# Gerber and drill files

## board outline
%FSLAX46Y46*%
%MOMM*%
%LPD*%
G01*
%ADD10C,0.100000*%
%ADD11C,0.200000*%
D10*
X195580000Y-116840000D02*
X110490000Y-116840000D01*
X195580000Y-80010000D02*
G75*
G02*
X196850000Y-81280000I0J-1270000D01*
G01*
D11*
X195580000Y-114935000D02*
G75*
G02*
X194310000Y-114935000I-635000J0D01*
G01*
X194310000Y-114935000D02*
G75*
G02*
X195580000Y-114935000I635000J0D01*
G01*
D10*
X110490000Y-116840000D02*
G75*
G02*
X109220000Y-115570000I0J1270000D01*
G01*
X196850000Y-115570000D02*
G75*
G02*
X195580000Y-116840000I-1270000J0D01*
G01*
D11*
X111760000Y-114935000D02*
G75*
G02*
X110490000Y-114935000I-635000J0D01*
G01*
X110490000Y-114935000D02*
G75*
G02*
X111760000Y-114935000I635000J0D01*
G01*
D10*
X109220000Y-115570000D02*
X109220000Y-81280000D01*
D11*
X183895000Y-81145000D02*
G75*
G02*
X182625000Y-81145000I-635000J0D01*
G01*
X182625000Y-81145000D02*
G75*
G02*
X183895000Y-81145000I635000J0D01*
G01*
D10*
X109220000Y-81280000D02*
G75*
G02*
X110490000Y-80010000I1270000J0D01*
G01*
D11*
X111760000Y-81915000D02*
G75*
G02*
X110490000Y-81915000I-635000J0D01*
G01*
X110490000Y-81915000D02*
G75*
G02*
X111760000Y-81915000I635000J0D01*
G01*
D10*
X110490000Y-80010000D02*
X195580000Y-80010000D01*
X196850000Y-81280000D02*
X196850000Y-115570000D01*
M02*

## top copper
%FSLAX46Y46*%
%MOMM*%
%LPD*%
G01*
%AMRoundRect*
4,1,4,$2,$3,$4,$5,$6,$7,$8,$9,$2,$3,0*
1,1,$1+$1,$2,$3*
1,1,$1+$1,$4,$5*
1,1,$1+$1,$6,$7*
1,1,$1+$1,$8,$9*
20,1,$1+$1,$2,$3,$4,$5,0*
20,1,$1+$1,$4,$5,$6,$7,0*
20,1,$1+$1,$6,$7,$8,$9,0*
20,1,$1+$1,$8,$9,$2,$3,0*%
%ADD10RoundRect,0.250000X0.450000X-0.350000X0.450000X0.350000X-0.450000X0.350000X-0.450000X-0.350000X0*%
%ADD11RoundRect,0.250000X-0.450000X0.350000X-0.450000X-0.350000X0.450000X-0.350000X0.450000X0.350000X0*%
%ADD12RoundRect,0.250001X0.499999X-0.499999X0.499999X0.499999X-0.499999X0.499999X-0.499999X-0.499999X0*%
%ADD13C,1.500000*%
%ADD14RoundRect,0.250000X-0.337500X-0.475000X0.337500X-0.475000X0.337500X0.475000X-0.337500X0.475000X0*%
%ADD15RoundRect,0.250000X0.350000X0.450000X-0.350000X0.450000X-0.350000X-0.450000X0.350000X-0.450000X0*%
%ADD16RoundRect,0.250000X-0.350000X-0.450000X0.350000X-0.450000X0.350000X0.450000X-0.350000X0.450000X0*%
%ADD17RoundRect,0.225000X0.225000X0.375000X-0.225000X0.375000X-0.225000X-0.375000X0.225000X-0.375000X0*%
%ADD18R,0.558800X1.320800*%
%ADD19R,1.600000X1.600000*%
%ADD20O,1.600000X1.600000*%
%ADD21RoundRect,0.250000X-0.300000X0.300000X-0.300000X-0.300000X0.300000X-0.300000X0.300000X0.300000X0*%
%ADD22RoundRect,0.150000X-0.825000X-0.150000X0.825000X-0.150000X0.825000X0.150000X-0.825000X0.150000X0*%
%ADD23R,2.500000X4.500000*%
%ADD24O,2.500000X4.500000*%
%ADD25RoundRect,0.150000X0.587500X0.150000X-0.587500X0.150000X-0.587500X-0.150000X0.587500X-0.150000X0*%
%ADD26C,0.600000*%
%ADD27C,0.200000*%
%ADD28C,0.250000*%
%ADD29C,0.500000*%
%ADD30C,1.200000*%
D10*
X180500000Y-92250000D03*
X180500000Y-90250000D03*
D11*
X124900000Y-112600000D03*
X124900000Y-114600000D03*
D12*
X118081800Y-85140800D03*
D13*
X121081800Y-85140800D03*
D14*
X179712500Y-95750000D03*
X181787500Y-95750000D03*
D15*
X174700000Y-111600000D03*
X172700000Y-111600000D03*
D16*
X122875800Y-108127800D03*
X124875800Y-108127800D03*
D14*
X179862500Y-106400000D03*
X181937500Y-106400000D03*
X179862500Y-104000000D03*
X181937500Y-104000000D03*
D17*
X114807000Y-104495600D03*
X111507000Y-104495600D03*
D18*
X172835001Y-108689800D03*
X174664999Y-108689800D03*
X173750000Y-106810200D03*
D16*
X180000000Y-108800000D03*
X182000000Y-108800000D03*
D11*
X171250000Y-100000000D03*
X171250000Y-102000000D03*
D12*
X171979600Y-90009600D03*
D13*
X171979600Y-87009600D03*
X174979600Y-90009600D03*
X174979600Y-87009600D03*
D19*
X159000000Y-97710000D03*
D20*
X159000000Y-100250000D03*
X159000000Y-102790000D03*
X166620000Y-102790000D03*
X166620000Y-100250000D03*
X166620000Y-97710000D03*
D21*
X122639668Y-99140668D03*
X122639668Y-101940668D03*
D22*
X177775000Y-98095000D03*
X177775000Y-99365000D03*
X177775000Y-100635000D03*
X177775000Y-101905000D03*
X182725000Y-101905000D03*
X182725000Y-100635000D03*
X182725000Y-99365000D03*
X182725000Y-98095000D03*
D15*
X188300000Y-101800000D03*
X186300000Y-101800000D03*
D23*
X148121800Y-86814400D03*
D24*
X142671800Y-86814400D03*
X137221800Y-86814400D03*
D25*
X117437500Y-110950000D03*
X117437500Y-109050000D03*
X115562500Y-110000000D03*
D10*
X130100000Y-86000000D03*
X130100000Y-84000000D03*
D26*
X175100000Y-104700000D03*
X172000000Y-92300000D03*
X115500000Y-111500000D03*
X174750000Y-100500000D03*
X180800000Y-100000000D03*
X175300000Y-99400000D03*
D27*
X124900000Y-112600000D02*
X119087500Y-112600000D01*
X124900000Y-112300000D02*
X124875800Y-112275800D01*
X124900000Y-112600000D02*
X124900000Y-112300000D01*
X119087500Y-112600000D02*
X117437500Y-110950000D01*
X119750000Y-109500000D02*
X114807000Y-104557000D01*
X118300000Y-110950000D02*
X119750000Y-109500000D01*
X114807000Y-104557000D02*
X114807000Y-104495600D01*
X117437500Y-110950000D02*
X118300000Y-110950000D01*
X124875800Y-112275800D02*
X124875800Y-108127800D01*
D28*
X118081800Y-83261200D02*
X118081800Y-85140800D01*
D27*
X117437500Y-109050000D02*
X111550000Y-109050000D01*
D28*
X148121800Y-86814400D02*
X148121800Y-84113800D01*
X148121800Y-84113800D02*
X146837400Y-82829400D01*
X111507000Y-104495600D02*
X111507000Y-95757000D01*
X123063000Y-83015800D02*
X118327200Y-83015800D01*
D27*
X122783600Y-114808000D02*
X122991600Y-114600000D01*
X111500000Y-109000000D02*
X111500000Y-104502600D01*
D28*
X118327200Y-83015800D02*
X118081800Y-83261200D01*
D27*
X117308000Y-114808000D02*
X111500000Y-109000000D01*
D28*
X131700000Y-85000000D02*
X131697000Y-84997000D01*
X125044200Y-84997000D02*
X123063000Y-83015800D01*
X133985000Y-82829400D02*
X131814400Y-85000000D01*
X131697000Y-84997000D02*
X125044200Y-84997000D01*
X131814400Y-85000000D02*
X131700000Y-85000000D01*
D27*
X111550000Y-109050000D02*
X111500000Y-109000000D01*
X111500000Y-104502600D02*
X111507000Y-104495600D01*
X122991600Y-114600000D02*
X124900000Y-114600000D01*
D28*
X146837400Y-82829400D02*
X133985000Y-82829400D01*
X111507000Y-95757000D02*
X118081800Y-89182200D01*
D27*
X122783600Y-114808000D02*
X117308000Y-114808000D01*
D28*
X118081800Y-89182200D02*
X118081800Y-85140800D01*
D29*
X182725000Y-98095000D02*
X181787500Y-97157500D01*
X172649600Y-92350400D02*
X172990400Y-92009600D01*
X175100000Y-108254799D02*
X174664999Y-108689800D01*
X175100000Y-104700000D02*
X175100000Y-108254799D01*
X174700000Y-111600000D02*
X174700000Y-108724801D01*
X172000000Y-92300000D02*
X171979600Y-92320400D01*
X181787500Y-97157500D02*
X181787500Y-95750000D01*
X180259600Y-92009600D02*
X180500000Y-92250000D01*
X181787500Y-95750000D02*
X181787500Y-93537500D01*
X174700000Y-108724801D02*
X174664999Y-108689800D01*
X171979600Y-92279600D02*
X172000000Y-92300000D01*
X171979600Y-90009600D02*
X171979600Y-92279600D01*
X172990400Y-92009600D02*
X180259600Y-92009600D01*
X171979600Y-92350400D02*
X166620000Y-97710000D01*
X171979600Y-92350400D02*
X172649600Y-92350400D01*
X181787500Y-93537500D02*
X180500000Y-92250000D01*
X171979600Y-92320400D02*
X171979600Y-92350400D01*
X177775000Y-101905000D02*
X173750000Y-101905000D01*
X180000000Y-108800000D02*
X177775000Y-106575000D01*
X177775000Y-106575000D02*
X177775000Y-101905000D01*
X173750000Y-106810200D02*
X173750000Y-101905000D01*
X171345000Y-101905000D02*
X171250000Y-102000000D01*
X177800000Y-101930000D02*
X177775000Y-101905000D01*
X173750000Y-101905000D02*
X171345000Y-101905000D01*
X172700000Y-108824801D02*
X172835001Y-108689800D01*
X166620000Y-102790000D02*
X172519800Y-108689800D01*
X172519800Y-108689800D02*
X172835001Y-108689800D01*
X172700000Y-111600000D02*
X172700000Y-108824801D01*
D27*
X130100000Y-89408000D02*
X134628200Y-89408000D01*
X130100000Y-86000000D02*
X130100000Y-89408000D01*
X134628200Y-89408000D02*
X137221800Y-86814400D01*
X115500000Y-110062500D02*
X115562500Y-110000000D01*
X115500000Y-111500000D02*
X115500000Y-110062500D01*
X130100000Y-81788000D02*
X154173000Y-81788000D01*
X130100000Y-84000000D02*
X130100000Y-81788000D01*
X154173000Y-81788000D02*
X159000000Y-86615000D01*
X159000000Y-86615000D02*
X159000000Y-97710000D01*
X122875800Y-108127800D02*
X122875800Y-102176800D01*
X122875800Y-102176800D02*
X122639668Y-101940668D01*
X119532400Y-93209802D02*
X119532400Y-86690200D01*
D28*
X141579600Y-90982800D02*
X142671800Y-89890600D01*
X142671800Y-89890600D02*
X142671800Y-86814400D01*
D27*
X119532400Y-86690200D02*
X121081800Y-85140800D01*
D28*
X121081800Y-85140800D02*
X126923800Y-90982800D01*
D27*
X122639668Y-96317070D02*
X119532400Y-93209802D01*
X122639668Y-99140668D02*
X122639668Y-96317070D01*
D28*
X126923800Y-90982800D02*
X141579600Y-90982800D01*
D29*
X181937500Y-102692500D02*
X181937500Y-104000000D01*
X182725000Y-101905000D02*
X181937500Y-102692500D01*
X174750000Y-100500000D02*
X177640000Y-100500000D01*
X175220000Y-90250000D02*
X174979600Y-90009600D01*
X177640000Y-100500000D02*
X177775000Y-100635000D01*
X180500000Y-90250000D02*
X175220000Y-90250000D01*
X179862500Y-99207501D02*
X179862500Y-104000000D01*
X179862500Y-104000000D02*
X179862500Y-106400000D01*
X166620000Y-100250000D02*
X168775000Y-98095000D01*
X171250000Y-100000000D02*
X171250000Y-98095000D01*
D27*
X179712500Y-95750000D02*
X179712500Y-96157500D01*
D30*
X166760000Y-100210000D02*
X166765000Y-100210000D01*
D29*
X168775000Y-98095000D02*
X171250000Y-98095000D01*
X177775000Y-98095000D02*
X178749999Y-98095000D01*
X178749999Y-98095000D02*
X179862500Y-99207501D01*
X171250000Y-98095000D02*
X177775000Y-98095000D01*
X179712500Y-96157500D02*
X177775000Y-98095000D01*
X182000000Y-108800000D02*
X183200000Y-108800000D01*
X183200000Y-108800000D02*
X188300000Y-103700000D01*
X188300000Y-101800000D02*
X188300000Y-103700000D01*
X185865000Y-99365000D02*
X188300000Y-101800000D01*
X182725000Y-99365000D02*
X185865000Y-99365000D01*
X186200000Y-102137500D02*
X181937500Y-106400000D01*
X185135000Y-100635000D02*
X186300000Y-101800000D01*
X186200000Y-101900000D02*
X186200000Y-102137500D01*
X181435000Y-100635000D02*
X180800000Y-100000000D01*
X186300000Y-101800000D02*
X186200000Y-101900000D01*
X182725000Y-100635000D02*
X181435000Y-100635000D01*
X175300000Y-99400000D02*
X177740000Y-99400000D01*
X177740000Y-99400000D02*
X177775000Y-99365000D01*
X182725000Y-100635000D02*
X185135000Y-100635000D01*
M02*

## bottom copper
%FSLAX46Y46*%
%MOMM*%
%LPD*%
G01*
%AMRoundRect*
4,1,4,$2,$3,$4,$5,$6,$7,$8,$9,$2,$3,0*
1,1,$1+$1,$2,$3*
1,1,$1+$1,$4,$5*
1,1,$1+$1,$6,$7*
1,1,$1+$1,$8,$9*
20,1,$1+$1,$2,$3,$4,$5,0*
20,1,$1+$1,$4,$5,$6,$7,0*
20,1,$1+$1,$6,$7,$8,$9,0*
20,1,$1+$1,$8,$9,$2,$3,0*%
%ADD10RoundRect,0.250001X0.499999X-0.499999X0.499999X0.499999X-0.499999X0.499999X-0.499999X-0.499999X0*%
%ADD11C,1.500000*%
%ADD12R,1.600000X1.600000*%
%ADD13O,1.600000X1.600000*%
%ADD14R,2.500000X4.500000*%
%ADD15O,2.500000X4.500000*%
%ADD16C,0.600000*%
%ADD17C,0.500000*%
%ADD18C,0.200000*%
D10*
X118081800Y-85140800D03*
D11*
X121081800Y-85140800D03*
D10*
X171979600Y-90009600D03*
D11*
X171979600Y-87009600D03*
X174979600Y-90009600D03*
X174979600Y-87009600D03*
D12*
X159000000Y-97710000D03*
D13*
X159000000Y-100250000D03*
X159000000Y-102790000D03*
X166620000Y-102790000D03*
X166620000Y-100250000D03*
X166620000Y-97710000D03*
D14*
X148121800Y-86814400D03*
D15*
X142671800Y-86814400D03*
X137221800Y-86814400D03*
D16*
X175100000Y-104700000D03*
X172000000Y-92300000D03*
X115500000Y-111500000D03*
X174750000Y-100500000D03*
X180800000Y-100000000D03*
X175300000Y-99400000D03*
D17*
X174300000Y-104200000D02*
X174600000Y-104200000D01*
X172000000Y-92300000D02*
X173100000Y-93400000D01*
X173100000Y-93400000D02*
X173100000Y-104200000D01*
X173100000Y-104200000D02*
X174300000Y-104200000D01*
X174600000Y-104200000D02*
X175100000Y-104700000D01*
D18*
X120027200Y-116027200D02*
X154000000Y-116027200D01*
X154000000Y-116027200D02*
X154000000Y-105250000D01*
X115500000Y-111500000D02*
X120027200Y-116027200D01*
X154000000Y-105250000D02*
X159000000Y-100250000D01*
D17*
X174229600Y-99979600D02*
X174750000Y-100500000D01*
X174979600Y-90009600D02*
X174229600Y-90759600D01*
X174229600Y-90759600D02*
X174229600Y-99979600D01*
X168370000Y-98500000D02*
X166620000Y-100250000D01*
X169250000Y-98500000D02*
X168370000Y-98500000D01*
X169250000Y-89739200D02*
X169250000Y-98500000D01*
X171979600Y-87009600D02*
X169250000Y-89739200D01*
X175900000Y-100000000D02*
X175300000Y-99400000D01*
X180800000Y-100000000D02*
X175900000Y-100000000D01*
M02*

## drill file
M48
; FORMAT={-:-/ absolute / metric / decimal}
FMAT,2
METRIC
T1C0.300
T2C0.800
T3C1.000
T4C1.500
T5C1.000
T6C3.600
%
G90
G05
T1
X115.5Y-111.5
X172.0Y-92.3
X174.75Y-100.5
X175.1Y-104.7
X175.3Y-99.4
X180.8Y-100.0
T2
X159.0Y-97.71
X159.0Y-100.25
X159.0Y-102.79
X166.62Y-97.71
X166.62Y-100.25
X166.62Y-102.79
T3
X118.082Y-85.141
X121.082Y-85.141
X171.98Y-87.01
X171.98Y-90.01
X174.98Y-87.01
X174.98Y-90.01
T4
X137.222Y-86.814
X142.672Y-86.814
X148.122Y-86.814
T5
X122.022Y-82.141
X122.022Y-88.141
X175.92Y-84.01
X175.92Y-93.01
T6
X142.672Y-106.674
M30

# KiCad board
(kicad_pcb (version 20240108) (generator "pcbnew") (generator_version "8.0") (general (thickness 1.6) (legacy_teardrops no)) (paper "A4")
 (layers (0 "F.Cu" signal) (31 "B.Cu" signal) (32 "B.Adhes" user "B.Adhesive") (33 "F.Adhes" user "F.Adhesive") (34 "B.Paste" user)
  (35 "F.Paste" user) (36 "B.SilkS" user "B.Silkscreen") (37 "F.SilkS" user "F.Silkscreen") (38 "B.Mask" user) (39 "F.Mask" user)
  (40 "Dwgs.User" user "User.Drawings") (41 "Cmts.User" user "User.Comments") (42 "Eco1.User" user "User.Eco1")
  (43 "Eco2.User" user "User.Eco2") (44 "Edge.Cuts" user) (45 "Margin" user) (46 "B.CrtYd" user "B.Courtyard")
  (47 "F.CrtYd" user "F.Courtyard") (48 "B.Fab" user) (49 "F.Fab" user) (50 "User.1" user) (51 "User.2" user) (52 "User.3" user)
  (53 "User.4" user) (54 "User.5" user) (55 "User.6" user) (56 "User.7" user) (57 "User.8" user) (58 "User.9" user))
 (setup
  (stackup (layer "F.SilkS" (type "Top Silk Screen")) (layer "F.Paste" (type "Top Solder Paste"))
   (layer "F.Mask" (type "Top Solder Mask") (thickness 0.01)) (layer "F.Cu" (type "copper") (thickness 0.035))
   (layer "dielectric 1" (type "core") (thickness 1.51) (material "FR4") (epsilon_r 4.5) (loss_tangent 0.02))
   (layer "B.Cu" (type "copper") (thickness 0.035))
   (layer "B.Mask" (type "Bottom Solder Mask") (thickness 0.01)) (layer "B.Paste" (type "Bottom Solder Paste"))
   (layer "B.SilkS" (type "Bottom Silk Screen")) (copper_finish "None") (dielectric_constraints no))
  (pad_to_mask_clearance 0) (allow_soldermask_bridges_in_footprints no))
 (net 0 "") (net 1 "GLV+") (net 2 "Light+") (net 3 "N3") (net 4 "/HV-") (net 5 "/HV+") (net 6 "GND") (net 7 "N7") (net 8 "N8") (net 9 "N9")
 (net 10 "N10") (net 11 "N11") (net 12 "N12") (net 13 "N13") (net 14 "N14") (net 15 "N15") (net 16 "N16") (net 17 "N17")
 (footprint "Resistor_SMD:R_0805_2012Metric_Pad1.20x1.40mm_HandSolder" (layer "F.Cu") (at 180.5 91.25 90)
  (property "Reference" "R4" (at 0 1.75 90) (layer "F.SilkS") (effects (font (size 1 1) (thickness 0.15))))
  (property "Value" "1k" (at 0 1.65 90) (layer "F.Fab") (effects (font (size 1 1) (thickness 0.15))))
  (pad "1" smd roundrect (at -1 0 90) (size 1.2 1.4) (layers "F.Cu" "F.Paste" "F.Mask") (roundrect_rratio 0.208333) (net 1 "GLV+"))
  (pad "2" smd roundrect (at 1 0 90) (size 1.2 1.4) (layers "F.Cu" "F.Paste" "F.Mask") (roundrect_rratio 0.208333) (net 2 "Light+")))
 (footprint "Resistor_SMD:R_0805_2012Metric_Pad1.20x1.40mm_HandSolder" (layer "F.Cu") (at 124.9 113.6 -90)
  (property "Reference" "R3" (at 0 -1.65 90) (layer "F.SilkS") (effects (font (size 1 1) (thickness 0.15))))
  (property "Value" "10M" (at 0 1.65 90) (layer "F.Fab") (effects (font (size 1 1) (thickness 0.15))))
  (pad "1" smd roundrect (at -1 0 270) (size 1.2 1.4) (layers "F.Cu" "F.Paste" "F.Mask") (roundrect_rratio 0.208333) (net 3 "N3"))
  (pad "2" smd roundrect (at 1 0 270) (size 1.2 1.4) (layers "F.Cu" "F.Paste" "F.Mask") (roundrect_rratio 0.208333) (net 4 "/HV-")))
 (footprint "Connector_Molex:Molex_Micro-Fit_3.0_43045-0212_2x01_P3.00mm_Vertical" (layer "F.Cu") (at 118.0818 85.1408 90)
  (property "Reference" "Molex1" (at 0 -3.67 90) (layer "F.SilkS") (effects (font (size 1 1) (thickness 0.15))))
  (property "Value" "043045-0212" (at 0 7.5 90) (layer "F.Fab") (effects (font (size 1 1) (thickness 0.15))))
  (pad "" np_thru_hole circle (at -3 3.94 90) (size 1 1) (drill 1) (layers "*.Cu" "*.Mask"))
  (pad "" np_thru_hole circle (at 3 3.94 90) (size 1 1) (drill 1) (layers "*.Cu" "*.Mask"))
  (pad "1" thru_hole roundrect (at 0 0 90) (size 1.5 1.5) (drill 1) (layers "*.Cu" "*.Mask") (remove_unused_layers no)
   (roundrect_rratio 0.166667) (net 4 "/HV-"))
  (pad "2" thru_hole circle (at 0 3 90) (size 1.5 1.5) (drill 1) (layers "*.Cu" "*.Mask") (remove_unused_layers no) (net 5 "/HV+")))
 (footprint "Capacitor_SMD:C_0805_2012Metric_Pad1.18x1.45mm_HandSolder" (layer "F.Cu") (at 180.75 95.75)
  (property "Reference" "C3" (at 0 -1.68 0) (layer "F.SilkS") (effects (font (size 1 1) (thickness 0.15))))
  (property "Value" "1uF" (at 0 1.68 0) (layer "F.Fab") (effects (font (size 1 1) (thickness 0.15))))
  (pad "1" smd roundrect (at -1.0375 0) (size 1.175 1.45) (layers "F.Cu" "F.Paste" "F.Mask") (roundrect_rratio 0.212766) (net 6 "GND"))
  (pad "2" smd roundrect (at 1.0375 0) (size 1.175 1.45) (layers "F.Cu" "F.Paste" "F.Mask") (roundrect_rratio 0.212766) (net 1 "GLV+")))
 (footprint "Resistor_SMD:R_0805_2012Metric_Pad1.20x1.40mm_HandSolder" (layer "F.Cu") (at 173.7 111.6 180)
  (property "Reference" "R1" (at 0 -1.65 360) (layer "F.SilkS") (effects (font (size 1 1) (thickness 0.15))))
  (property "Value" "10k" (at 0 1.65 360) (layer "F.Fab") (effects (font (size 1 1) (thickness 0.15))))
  (pad "1" smd roundrect (at -1 0 180) (size 1.2 1.4) (layers "F.Cu" "F.Paste" "F.Mask") (roundrect_rratio 0.208333) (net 1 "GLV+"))
  (pad "2" smd roundrect (at 1 0 180) (size 1.2 1.4) (layers "F.Cu" "F.Paste" "F.Mask") (roundrect_rratio 0.208333) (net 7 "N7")))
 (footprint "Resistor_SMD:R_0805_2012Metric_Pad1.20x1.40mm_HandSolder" (layer "F.Cu") (at 123.8758 108.1278)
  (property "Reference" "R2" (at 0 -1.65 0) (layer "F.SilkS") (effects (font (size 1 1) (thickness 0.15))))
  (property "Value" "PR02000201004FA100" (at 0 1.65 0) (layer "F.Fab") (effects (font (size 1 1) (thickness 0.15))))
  (pad "1" smd roundrect (at -1 0) (size 1.2 1.4) (layers "F.Cu" "F.Paste" "F.Mask") (roundrect_rratio 0.208333) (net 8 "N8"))
  (pad "2" smd roundrect (at 1 0) (size 1.2 1.4) (layers "F.Cu" "F.Paste" "F.Mask") (roundrect_rratio 0.208333) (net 3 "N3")))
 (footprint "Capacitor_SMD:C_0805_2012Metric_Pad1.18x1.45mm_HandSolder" (layer "F.Cu") (at 180.9 106.4)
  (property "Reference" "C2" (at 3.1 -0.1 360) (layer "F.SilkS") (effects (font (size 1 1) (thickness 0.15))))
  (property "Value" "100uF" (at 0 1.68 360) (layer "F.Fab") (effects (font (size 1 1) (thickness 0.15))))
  (pad "1" smd roundrect (at -1.0375 0) (size 1.175 1.45) (layers "F.Cu" "F.Paste" "F.Mask") (roundrect_rratio 0.212766) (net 6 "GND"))
  (pad "2" smd roundrect (at 1.0375 0) (size 1.175 1.45) (layers "F.Cu" "F.Paste" "F.Mask") (roundrect_rratio 0.212766) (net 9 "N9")))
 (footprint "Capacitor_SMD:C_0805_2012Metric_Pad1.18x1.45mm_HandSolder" (layer "F.Cu") (at 180.9 104)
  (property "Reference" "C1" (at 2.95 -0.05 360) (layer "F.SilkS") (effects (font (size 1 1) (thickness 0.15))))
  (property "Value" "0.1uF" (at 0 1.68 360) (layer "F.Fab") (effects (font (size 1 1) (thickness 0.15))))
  (pad "1" smd roundrect (at -1.0375 0) (size 1.175 1.45) (layers "F.Cu" "F.Paste" "F.Mask") (roundrect_rratio 0.212766) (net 6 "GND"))
  (pad "2" smd roundrect (at 1.0375 0) (size 1.175 1.45) (layers "F.Cu" "F.Paste" "F.Mask") (roundrect_rratio 0.212766) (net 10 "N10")))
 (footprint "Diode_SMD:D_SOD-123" (layer "F.Cu") (at 113.157 104.4956 180)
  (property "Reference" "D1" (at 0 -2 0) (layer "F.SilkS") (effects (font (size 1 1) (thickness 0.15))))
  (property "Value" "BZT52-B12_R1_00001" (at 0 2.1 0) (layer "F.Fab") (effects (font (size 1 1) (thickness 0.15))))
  (pad "1" smd roundrect (at -1.65 0 180) (size 0.9 1.2) (layers "F.Cu" "F.Paste" "F.Mask") (roundrect_rratio 0.25) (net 3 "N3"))
  (pad "2" smd roundrect (at 1.65 0 180) (size 0.9 1.2) (layers "F.Cu" "F.Paste" "F.Mask") (roundrect_rratio 0.25) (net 4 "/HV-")))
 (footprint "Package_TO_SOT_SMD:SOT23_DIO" (layer "F.Cu") (at 173.75 107.75)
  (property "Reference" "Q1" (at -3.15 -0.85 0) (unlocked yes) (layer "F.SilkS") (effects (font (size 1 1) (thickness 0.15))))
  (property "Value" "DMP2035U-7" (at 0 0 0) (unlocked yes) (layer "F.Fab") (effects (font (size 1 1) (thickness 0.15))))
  (pad "1" smd rect (at -0.914999 0.9398) (size 0.5588 1.3208) (layers "F.Cu" "F.Paste" "F.Mask") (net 7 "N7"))
  (pad "2" smd rect (at 0.914999 0.9398) (size 0.5588 1.3208) (layers "F.Cu" "F.Paste" "F.Mask") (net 1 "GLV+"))
  (pad "3" smd rect (at 0 -0.9398) (size 0.5588 1.3208) (layers "F.Cu" "F.Paste" "F.Mask") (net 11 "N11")))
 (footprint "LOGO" (layer "F.Cu") (at 156.25 108.5)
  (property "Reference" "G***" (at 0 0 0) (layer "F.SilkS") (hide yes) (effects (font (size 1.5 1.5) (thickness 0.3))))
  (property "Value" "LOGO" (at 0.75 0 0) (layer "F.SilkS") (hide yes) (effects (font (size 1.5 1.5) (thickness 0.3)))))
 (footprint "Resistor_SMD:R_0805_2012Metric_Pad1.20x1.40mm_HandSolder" (layer "F.Cu") (at 181 108.8)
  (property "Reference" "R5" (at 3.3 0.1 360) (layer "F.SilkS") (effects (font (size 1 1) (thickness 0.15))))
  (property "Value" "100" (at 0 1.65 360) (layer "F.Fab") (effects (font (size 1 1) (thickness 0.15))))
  (pad "1" smd roundrect (at -1 0) (size 1.2 1.4) (layers "F.Cu" "F.Paste" "F.Mask") (roundrect_rratio 0.208333) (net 11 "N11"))
  (pad "2" smd roundrect (at 1 0) (size 1.2 1.4) (layers "F.Cu" "F.Paste" "F.Mask") (roundrect_rratio 0.208333) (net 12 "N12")))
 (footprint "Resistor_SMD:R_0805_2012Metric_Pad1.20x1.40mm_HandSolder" (layer "F.Cu") (at 171.25 101 -90)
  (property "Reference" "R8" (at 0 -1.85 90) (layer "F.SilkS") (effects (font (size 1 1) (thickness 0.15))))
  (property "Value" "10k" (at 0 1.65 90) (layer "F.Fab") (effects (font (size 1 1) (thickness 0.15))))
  (pad "1" smd roundrect (at -1 0 270) (size 1.2 1.4) (layers "F.Cu" "F.Paste" "F.Mask") (roundrect_rratio 0.208333) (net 6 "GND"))
  (pad "2" smd roundrect (at 1 0 270) (size 1.2 1.4) (layers "F.Cu" "F.Paste" "F.Mask") (roundrect_rratio 0.208333) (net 11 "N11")))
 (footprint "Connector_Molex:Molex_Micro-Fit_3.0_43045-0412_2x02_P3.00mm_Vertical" (layer "F.Cu") (at 171.9796 90.0096 90)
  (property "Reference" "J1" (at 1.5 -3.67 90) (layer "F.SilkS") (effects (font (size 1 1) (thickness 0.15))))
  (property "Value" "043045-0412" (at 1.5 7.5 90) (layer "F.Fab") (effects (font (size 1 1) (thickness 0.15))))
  (pad "" np_thru_hole circle (at -3 3.94 90) (size 1 1) (drill 1) (layers "*.Cu" "*.Mask"))
  (pad "" np_thru_hole circle (at 6 3.94 90) (size 1 1) (drill 1) (layers "*.Cu" "*.Mask"))
  (pad "1" thru_hole roundrect (at 0 0 90) (size 1.5 1.5) (drill 1) (layers "*.Cu" "*.Mask") (remove_unused_layers no)
   (roundrect_rratio 0.166667) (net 1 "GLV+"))
  (pad "2" thru_hole circle (at 3 0 90) (size 1.5 1.5) (drill 1) (layers "*.Cu" "*.Mask") (remove_unused_layers no) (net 6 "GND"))
  (pad "3" thru_hole circle (at 0 3 90) (size 1.5 1.5) (drill 1) (layers "*.Cu" "*.Mask") (remove_unused_layers no) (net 2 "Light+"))
  (pad "4" thru_hole circle (at 3 3 90) (size 1.5 1.5) (drill 1) (layers "*.Cu" "*.Mask") (remove_unused_layers no) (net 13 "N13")))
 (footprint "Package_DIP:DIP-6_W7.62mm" (layer "F.Cu") (at 159 97.71)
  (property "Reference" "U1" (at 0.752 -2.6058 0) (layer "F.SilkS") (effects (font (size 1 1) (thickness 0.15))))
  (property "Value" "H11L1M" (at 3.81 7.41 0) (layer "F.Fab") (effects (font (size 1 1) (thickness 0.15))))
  (pad "1" thru_hole rect (at 0 0) (size 1.6 1.6) (drill 0.8) (layers "*.Cu" "*.Mask") (remove_unused_layers no) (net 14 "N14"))
  (pad "2" thru_hole oval (at 0 2.54) (size 1.6 1.6) (drill 0.8) (layers "*.Cu" "*.Mask") (remove_unused_layers no) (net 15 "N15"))
  (pad "3" thru_hole oval (at 0 5.08) (size 1.6 1.6) (drill 0.8) (layers "*.Cu" "*.Mask") (remove_unused_layers no) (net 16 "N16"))
  (pad "4" thru_hole oval (at 7.62 5.08) (size 1.6 1.6) (drill 0.8) (layers "*.Cu" "*.Mask") (remove_unused_layers no) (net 7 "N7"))
  (pad "5" thru_hole oval (at 7.62 2.54) (size 1.6 1.6) (drill 0.8) (layers "*.Cu" "*.Mask") (remove_unused_layers no) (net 6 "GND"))
  (pad "6" thru_hole oval (at 7.62 0) (size 1.6 1.6) (drill 0.8) (layers "*.Cu" "*.Mask") (remove_unused_layers no) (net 1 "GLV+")))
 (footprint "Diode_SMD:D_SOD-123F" (layer "F.Cu") (at 122.639668 100.540668 -90)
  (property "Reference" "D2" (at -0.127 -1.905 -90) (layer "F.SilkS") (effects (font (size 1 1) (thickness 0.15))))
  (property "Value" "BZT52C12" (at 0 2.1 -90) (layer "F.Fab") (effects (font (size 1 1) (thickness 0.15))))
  (pad "1" smd roundrect (at -1.4 0 270) (size 1.1 1.1) (layers "F.Cu" "F.Paste" "F.Mask") (roundrect_rratio 0.2272727273) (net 5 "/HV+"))
  (pad "2" smd roundrect (at 1.4 0 270) (size 1.1 1.1) (layers "F.Cu" "F.Paste" "F.Mask") (roundrect_rratio 0.2272727273) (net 8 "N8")))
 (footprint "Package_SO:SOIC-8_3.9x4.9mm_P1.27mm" (layer "F.Cu") (at 180.25 100)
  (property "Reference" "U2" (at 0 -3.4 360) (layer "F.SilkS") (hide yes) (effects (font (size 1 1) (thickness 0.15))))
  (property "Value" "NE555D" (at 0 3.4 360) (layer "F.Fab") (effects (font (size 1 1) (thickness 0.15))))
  (pad "1" smd roundrect (at -2.475 -1.905) (size 1.95 0.6) (layers "F.Cu" "F.Paste" "F.Mask") (roundrect_rratio 0.25) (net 6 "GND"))
  (pad "2" smd roundrect (at -2.475 -0.635) (size 1.95 0.6) (layers "F.Cu" "F.Paste" "F.Mask") (roundrect_rratio 0.25) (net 9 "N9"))
  (pad "3" smd roundrect (at -2.475 0.635) (size 1.95 0.6) (layers "F.Cu" "F.Paste" "F.Mask") (roundrect_rratio 0.25) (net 2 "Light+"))
  (pad "4" smd roundrect (at -2.475 1.905) (size 1.95 0.6) (layers "F.Cu" "F.Paste" "F.Mask") (roundrect_rratio 0.25) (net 11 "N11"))
  (pad "5" smd roundrect (at 2.475 1.905) (size 1.95 0.6) (layers "F.Cu" "F.Paste" "F.Mask") (roundrect_rratio 0.25) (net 10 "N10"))
  (pad "6" smd roundrect (at 2.475 0.635) (size 1.95 0.6) (layers "F.Cu" "F.Paste" "F.Mask") (roundrect_rratio 0.25) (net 9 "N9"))
  (pad "7" smd roundrect (at 2.475 -0.635) (size 1.95 0.6) (layers "F.Cu" "F.Paste" "F.Mask") (roundrect_rratio 0.25) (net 12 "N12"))
  (pad "8" smd roundrect (at 2.475 -1.905) (size 1.95 0.6) (layers "F.Cu" "F.Paste" "F.Mask") (roundrect_rratio 0.25) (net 1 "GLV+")))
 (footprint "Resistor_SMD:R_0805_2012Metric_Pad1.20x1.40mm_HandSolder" (layer "F.Cu") (at 187.3 101.8 180)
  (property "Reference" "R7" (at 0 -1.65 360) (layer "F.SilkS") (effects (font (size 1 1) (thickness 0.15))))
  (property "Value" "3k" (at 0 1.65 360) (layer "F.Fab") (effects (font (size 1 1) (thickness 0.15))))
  (pad "1" smd roundrect (at -1 0 180) (size 1.2 1.4) (layers "F.Cu" "F.Paste" "F.Mask") (roundrect_rratio 0.208333) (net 12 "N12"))
  (pad "2" smd roundrect (at 1 0 180) (size 1.2 1.4) (layers "F.Cu" "F.Paste" "F.Mask") (roundrect_rratio 0.208333) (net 9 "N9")))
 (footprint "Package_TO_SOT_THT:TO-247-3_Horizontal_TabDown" (layer "F.Cu") (at 148.1218 86.8144 180)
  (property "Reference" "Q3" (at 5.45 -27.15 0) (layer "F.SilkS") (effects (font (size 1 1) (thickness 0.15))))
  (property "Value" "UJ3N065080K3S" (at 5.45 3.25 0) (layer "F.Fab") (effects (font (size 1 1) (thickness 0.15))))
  (pad "" np_thru_hole oval (at 5.45 -19.86 180) (size 3.6 3.6) (drill 3.6) (layers "*.Cu" "*.Mask"))
  (pad "1" thru_hole rect (at 0 0 180) (size 2.5 4.5) (drill 1.5) (layers "*.Cu" "*.Mask") (remove_unused_layers no) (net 4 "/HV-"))
  (pad "2" thru_hole oval (at 5.45 0 180) (size 2.5 4.5) (drill 1.5) (layers "*.Cu" "*.Mask") (remove_unused_layers no) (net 5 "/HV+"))
  (pad "3" thru_hole oval (at 10.9 0 180) (size 2.5 4.5) (drill 1.5) (layers "*.Cu" "*.Mask") (remove_unused_layers no) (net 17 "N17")))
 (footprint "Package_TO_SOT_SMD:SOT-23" (layer "F.Cu") (at 116.5 110 180)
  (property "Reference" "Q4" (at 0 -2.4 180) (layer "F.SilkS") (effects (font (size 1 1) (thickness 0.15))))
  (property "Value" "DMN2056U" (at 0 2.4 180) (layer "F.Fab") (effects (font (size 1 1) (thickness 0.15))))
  (pad "1" smd roundrect (at -0.9375 -0.95 180) (size 1.475 0.6) (layers "F.Cu" "F.Paste" "F.Mask") (roundrect_rratio 0.25) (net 3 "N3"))
  (pad "2" smd roundrect (at -0.9375 0.95 180) (size 1.475 0.6) (layers "F.Cu" "F.Paste" "F.Mask") (roundrect_rratio 0.25) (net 4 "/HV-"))
  (pad "3" smd roundrect (at 0.9375 0 180) (size 1.475 0.6) (layers "F.Cu" "F.Paste" "F.Mask") (roundrect_rratio 0.25) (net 15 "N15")))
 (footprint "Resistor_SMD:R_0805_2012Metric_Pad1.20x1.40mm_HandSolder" (layer "F.Cu") (at 130.1 85 90)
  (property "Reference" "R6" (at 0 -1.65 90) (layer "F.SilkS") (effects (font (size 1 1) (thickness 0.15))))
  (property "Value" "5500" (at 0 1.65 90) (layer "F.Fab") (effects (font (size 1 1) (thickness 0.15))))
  (pad "1" smd roundrect (at -1 0 90) (size 1.2 1.4) (layers "F.Cu" "F.Paste" "F.Mask") (roundrect_rratio 0.208333) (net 17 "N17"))
  (pad "2" smd roundrect (at 1 0 90) (size 1.2 1.4) (layers "F.Cu" "F.Paste" "F.Mask") (roundrect_rratio 0.208333) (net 14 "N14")))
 (gr_line (start 195.58 116.84) (end 110.49 116.84) (stroke (width 0.1) (type default)) (layer "Edge.Cuts"))
 (gr_arc (start 195.58 80.01) (mid 196.478026 80.381974) (end 196.85 81.28) (stroke (width 0.1) (type default)) (layer "Edge.Cuts"))
 (gr_circle (center 194.945 114.935) (end 195.58 114.935) (stroke (width 0.2) (type default)) (fill none) (layer "Edge.Cuts"))
 (gr_arc (start 110.49 116.84) (mid 109.591974 116.468026) (end 109.22 115.57) (stroke (width 0.1) (type default)) (layer "Edge.Cuts"))
 (gr_arc (start 196.85 115.57) (mid 196.478026 116.468026) (end 195.58 116.84) (stroke (width 0.1) (type default)) (layer "Edge.Cuts"))
 (gr_circle (center 111.125 114.935) (end 111.76 114.935) (stroke (width 0.2) (type default)) (fill none) (layer "Edge.Cuts"))
 (gr_line (start 109.22 115.57) (end 109.22 81.28) (stroke (width 0.1) (type default)) (layer "Edge.Cuts"))
 (gr_circle (center 183.26 81.145) (end 183.895 81.145) (stroke (width 0.2) (type default)) (fill none) (layer "Edge.Cuts"))
 (gr_arc (start 109.22 81.28) (mid 109.591974 80.381974) (end 110.49 80.01) (stroke (width 0.1) (type default)) (layer "Edge.Cuts"))
 (gr_circle (center 111.125 81.915) (end 111.76 81.915) (stroke (width 0.2) (type default)) (fill none) (layer "Edge.Cuts"))
 (gr_line (start 110.49 80.01) (end 195.58 80.01) (stroke (width 0.1) (type default)) (layer "Edge.Cuts"))
 (gr_line (start 196.85 81.28) (end 196.85 115.57) (stroke (width 0.1) (type default)) (layer "Edge.Cuts"))
 (segment (start 124.9 112.6) (end 119.0875 112.6) (width 0.2) (layer "F.Cu") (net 3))
 (segment (start 124.9 112.3) (end 124.8758 112.2758) (width 0.2) (layer "F.Cu") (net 3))
 (segment (start 124.9 112.6) (end 124.9 112.3) (width 0.2) (layer "F.Cu") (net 3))
 (segment (start 119.0875 112.6) (end 117.4375 110.95) (width 0.2) (layer "F.Cu") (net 3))
 (segment (start 119.75 109.5) (end 114.807 104.557) (width 0.2) (layer "F.Cu") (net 3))
 (segment (start 118.3 110.95) (end 119.75 109.5) (width 0.2) (layer "F.Cu") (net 3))
 (segment (start 114.807 104.557) (end 114.807 104.4956) (width 0.2) (layer "F.Cu") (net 3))
 (segment (start 117.4375 110.95) (end 118.3 110.95) (width 0.2) (layer "F.Cu") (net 3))
 (segment (start 124.8758 112.2758) (end 124.8758 108.1278) (width 0.2) (layer "F.Cu") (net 3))
 (segment (start 118.0818 83.2612) (end 118.0818 85.1408) (width 0.25) (layer "F.Cu") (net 4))
 (segment (start 117.4375 109.05) (end 111.55 109.05) (width 0.2) (layer "F.Cu") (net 4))
 (segment (start 148.1218 86.8144) (end 148.1218 84.1138) (width 0.25) (layer "F.Cu") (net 4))
 (segment (start 148.1218 84.1138) (end 146.8374 82.8294) (width 0.25) (layer "F.Cu") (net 4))
 (segment (start 111.507 104.4956) (end 111.507 95.757) (width 0.25) (layer "F.Cu") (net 4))
 (segment (start 123.063 83.0158) (end 118.3272 83.0158) (width 0.25) (layer "F.Cu") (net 4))
 (segment (start 122.7836 114.808) (end 122.9916 114.6) (width 0.2) (layer "F.Cu") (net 4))
 (segment (start 111.5 109) (end 111.5 104.5026) (width 0.2) (layer "F.Cu") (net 4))
 (segment (start 118.3272 83.0158) (end 118.0818 83.2612) (width 0.25) (layer "F.Cu") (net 4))
 (segment (start 117.308 114.808) (end 111.5 109) (width 0.2) (layer "F.Cu") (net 4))
 (segment (start 131.7 85) (end 131.697 84.997) (width 0.25) (layer "F.Cu") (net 4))
 (segment (start 125.0442 84.997) (end 123.063 83.0158) (width 0.25) (layer "F.Cu") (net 4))
 (segment (start 133.985 82.8294) (end 131.8144 85) (width 0.25) (layer "F.Cu") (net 4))
 (segment (start 131.697 84.997) (end 125.0442 84.997) (width 0.25) (layer "F.Cu") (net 4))
 (segment (start 131.8144 85) (end 131.7 85) (width 0.25) (layer "F.Cu") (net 4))
 (segment (start 111.55 109.05) (end 111.5 109) (width 0.2) (layer "F.Cu") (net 4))
 (segment (start 111.5 104.5026) (end 111.507 104.4956) (width 0.2) (layer "F.Cu") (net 4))
 (segment (start 122.9916 114.6) (end 124.9 114.6) (width 0.2) (layer "F.Cu") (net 4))
 (segment (start 146.8374 82.8294) (end 133.985 82.8294) (width 0.25) (layer "F.Cu") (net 4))
 (segment (start 111.507 95.757) (end 118.0818 89.1822) (width 0.25) (layer "F.Cu") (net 4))
 (segment (start 122.7836 114.808) (end 117.308 114.808) (width 0.2) (layer "F.Cu") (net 4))
 (segment (start 118.0818 89.1822) (end 118.0818 85.1408) (width 0.25) (layer "F.Cu") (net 4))
 (segment (start 182.725 98.095) (end 181.7875 97.1575) (width 0.5) (layer "F.Cu") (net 1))
 (segment (start 172.6496 92.3504) (end 172.9904 92.0096) (width 0.5) (layer "F.Cu") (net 1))
 (segment (start 175.1 108.254799) (end 174.664999 108.6898) (width 0.5) (layer "F.Cu") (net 1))
 (segment (start 175.1 104.7) (end 175.1 108.254799) (width 0.5) (layer "F.Cu") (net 1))
 (segment (start 174.7 111.6) (end 174.7 108.724801) (width 0.5) (layer "F.Cu") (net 1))
 (segment (start 172 92.3) (end 171.9796 92.3204) (width 0.5) (layer "F.Cu") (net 1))
 (segment (start 181.7875 97.1575) (end 181.7875 95.75) (width 0.5) (layer "F.Cu") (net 1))
 (segment (start 180.2596 92.0096) (end 180.5 92.25) (width 0.5) (layer "F.Cu") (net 1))
 (segment (start 181.7875 95.75) (end 181.7875 93.5375) (width 0.5) (layer "F.Cu") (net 1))
 (segment (start 174.7 108.724801) (end 174.664999 108.6898) (width 0.5) (layer "F.Cu") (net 1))
 (segment (start 171.9796 92.2796) (end 172 92.3) (width 0.5) (layer "F.Cu") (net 1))
 (segment (start 171.9796 90.0096) (end 171.9796 92.2796) (width 0.5) (layer "F.Cu") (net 1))
 (segment (start 172.9904 92.0096) (end 180.2596 92.0096) (width 0.5) (layer "F.Cu") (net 1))
 (segment (start 171.9796 92.3504) (end 166.62 97.71) (width 0.5) (layer "F.Cu") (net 1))
 (segment (start 171.9796 92.3504) (end 172.6496 92.3504) (width 0.5) (layer "F.Cu") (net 1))
 (segment (start 181.7875 93.5375) (end 180.5 92.25) (width 0.5) (layer "F.Cu") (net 1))
 (segment (start 171.9796 92.3204) (end 171.9796 92.3504) (width 0.5) (layer "F.Cu") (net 1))
 (via (at 175.1 104.7) (size 0.6) (drill 0.3) (layers "F.Cu" "B.Cu") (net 1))
 (via (at 172 92.3) (size 0.6) (drill 0.3) (layers "F.Cu" "B.Cu") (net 1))
 (segment (start 174.3 104.2) (end 174.6 104.2) (width 0.5) (layer "B.Cu") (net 1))
 (segment (start 172 92.3) (end 173.1 93.4) (width 0.5) (layer "B.Cu") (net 1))
 (segment (start 173.1 93.4) (end 173.1 104.2) (width 0.5) (layer "B.Cu") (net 1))
 (segment (start 173.1 104.2) (end 174.3 104.2) (width 0.5) (layer "B.Cu") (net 1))
 (segment (start 174.6 104.2) (end 175.1 104.7) (width 0.5) (layer "B.Cu") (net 1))
 (segment (start 177.775 101.905) (end 173.75 101.905) (width 0.5) (layer "F.Cu") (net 11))
 (segment (start 180 108.8) (end 177.775 106.575) (width 0.5) (layer "F.Cu") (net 11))
 (segment (start 177.775 106.575) (end 177.775 101.905) (width 0.5) (layer "F.Cu") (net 11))
 (segment (start 173.75 106.8102) (end 173.75 101.905) (width 0.5) (layer "F.Cu") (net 11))
 (segment (start 171.345 101.905) (end 171.25 102) (width 0.5) (layer "F.Cu") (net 11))
 (segment (start 177.8 101.93) (end 177.775 101.905) (width 0.5) (layer "F.Cu") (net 11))
 (segment (start 173.75 101.905) (end 171.345 101.905) (width 0.5) (layer "F.Cu") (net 11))
 (segment (start 172.7 108.824801) (end 172.835001 108.6898) (width 0.5) (layer "F.Cu") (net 7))
 (segment (start 166.62 102.79) (end 172.5198 108.6898) (width 0.5) (layer "F.Cu") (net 7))
 (segment (start 172.5198 108.6898) (end 172.835001 108.6898) (width 0.5) (layer "F.Cu") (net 7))
 (segment (start 172.7 111.6) (end 172.7 108.824801) (width 0.5) (layer "F.Cu") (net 7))
 (segment (start 130.1 89.408) (end 134.6282 89.408) (width 0.2) (layer "F.Cu") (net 17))
 (segment (start 130.1 86) (end 130.1 89.408) (width 0.2) (layer "F.Cu") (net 17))
 (segment (start 134.6282 89.408) (end 137.2218 86.8144) (width 0.2) (layer "F.Cu") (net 17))
 (segment (start 115.5 110.0625) (end 115.5625 110) (width 0.2) (layer "F.Cu") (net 15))
 (segment (start 115.5 111.5) (end 115.5 110.0625) (width 0.2) (layer "F.Cu") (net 15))
 (via (at 115.5 111.5) (size 0.6) (drill 0.3) (layers "F.Cu" "B.Cu") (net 15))
 (segment (start 120.0272 116.0272) (end 154 116.0272) (width 0.2) (layer "B.Cu") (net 15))
 (segment (start 154 116.0272) (end 154 105.25) (width 0.2) (layer "B.Cu") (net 15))
 (segment (start 115.5 111.5) (end 120.0272 116.0272) (width 0.2) (layer "B.Cu") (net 15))
 (segment (start 154 105.25) (end 159 100.25) (width 0.2) (layer "B.Cu") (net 15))
 (segment (start 130.1 81.788) (end 154.173 81.788) (width 0.2) (layer "F.Cu") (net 14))
 (segment (start 130.1 84) (end 130.1 81.788) (width 0.2) (layer "F.Cu") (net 14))
 (segment (start 154.173 81.788) (end 159 86.615) (width 0.2) (layer "F.Cu") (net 14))
 (segment (start 159 86.615) (end 159 97.71) (width 0.2) (layer "F.Cu") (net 14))
 (segment (start 122.8758 108.1278) (end 122.8758 102.1768) (width 0.2) (layer "F.Cu") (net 8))
 (segment (start 122.8758 102.1768) (end 122.639668 101.940668) (width 0.2) (layer "F.Cu") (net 8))
 (segment (start 119.5324 93.209802) (end 119.5324 86.6902) (width 0.2) (layer "F.Cu") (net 5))
 (segment (start 141.5796 90.9828) (end 142.6718 89.8906) (width 0.25) (layer "F.Cu") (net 5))
 (segment (start 142.6718 89.8906) (end 142.6718 86.8144) (width 0.25) (layer "F.Cu") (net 5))
 (segment (start 119.5324 86.6902) (end 121.0818 85.1408) (width 0.2) (layer "F.Cu") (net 5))
 (segment (start 121.0818 85.1408) (end 126.9238 90.9828) (width 0.25) (layer "F.Cu") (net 5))
 (segment (start 122.639668 96.31707) (end 119.5324 93.209802) (width 0.2) (layer "F.Cu") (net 5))
 (segment (start 122.639668 99.140668) (end 122.639668 96.31707) (width 0.2) (layer "F.Cu") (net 5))
 (segment (start 126.9238 90.9828) (end 141.5796 90.9828) (width 0.25) (layer "F.Cu") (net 5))
 (segment (start 181.9375 102.6925) (end 181.9375 104) (width 0.5) (layer "F.Cu") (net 10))
 (segment (start 182.725 101.905) (end 181.9375 102.6925) (width 0.5) (layer "F.Cu") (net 10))
 (segment (start 174.75 100.5) (end 177.64 100.5) (width 0.5) (layer "F.Cu") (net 2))
 (segment (start 175.22 90.25) (end 174.9796 90.0096) (width 0.5) (layer "F.Cu") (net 2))
 (segment (start 177.64 100.5) (end 177.775 100.635) (width 0.5) (layer "F.Cu") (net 2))
 (segment (start 180.5 90.25) (end 175.22 90.25) (width 0.5) (layer "F.Cu") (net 2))
 (via (at 174.75 100.5) (size 0.6) (drill 0.3) (layers "F.Cu" "B.Cu") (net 2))
 (segment (start 174.2296 99.9796) (end 174.75 100.5) (width 0.5) (layer "B.Cu") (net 2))
 (segment (start 174.9796 90.0096) (end 174.2296 90.7596) (width 0.5) (layer "B.Cu") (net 2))
 (segment (start 174.2296 90.7596) (end 174.2296 99.9796) (width 0.5) (layer "B.Cu") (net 2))
 (segment (start 179.8625 99.207501) (end 179.8625 104) (width 0.5) (layer "F.Cu") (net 6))
 (segment (start 179.8625 104) (end 179.8625 106.4) (width 0.5) (layer "F.Cu") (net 6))
 (segment (start 166.62 100.25) (end 168.775 98.095) (width 0.5) (layer "F.Cu") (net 6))
 (segment (start 171.25 100) (end 171.25 98.095) (width 0.5) (layer "F.Cu") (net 6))
 (segment (start 179.7125 95.75) (end 179.7125 96.1575) (width 0.2) (layer "F.Cu") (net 6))
 (segment (start 166.76 100.21) (end 166.765 100.21) (width 1.2) (layer "F.Cu") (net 6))
 (segment (start 168.775 98.095) (end 171.25 98.095) (width 0.5) (layer "F.Cu") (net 6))
 (segment (start 177.775 98.095) (end 178.749999 98.095) (width 0.5) (layer "F.Cu") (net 6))
 (segment (start 178.749999 98.095) (end 179.8625 99.207501) (width 0.5) (layer "F.Cu") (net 6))
 (segment (start 171.25 98.095) (end 177.775 98.095) (width 0.5) (layer "F.Cu") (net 6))
 (segment (start 179.7125 96.1575) (end 177.775 98.095) (width 0.5) (layer "F.Cu") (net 6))
 (segment (start 168.37 98.5) (end 166.62 100.25) (width 0.5) (layer "B.Cu") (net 6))
 (segment (start 169.25 98.5) (end 168.37 98.5) (width 0.5) (layer "B.Cu") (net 6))
 (segment (start 169.25 89.7392) (end 169.25 98.5) (width 0.5) (layer "B.Cu") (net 6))
 (segment (start 171.9796 87.0096) (end 169.25 89.7392) (width 0.5) (layer "B.Cu") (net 6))
 (segment (start 182 108.8) (end 183.2 108.8) (width 0.5) (layer "F.Cu") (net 12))
 (segment (start 183.2 108.8) (end 188.3 103.7) (width 0.5) (layer "F.Cu") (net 12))
 (segment (start 188.3 101.8) (end 188.3 103.7) (width 0.5) (layer "F.Cu") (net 12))
 (segment (start 185.865 99.365) (end 188.3 101.8) (width 0.5) (layer "F.Cu") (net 12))
 (segment (start 182.725 99.365) (end 185.865 99.365) (width 0.5) (layer "F.Cu") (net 12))
 (segment (start 186.2 102.1375) (end 181.9375 106.4) (width 0.5) (layer "F.Cu") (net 9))
 (segment (start 185.135 100.635) (end 186.3 101.8) (width 0.5) (layer "F.Cu") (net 9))
 (segment (start 186.2 101.9) (end 186.2 102.1375) (width 0.5) (layer "F.Cu") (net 9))
 (segment (start 181.435 100.635) (end 180.8 100) (width 0.5) (layer "F.Cu") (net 9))
 (segment (start 186.3 101.8) (end 186.2 101.9) (width 0.5) (layer "F.Cu") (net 9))
 (segment (start 182.725 100.635) (end 181.435 100.635) (width 0.5) (layer "F.Cu") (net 9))
 (segment (start 175.3 99.4) (end 177.74 99.4) (width 0.5) (layer "F.Cu") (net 9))
 (segment (start 177.74 99.4) (end 177.775 99.365) (width 0.5) (layer "F.Cu") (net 9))
 (segment (start 182.725 100.635) (end 185.135 100.635) (width 0.5) (layer "F.Cu") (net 9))
 (via (at 180.8 100) (size 0.6) (drill 0.3) (layers "F.Cu" "B.Cu") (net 9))
 (via (at 175.3 99.4) (size 0.6) (drill 0.3) (layers "F.Cu" "B.Cu") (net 9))
 (segment (start 175.9 100) (end 175.3 99.4) (width 0.5) (layer "B.Cu") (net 9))
 (segment (start 180.8 100) (end 175.9 100) (width 0.5) (layer "B.Cu") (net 9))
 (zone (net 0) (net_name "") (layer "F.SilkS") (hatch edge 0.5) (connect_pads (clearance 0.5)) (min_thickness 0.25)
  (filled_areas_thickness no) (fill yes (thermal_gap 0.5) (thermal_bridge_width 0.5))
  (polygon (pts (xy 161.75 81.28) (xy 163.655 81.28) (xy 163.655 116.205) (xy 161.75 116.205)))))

